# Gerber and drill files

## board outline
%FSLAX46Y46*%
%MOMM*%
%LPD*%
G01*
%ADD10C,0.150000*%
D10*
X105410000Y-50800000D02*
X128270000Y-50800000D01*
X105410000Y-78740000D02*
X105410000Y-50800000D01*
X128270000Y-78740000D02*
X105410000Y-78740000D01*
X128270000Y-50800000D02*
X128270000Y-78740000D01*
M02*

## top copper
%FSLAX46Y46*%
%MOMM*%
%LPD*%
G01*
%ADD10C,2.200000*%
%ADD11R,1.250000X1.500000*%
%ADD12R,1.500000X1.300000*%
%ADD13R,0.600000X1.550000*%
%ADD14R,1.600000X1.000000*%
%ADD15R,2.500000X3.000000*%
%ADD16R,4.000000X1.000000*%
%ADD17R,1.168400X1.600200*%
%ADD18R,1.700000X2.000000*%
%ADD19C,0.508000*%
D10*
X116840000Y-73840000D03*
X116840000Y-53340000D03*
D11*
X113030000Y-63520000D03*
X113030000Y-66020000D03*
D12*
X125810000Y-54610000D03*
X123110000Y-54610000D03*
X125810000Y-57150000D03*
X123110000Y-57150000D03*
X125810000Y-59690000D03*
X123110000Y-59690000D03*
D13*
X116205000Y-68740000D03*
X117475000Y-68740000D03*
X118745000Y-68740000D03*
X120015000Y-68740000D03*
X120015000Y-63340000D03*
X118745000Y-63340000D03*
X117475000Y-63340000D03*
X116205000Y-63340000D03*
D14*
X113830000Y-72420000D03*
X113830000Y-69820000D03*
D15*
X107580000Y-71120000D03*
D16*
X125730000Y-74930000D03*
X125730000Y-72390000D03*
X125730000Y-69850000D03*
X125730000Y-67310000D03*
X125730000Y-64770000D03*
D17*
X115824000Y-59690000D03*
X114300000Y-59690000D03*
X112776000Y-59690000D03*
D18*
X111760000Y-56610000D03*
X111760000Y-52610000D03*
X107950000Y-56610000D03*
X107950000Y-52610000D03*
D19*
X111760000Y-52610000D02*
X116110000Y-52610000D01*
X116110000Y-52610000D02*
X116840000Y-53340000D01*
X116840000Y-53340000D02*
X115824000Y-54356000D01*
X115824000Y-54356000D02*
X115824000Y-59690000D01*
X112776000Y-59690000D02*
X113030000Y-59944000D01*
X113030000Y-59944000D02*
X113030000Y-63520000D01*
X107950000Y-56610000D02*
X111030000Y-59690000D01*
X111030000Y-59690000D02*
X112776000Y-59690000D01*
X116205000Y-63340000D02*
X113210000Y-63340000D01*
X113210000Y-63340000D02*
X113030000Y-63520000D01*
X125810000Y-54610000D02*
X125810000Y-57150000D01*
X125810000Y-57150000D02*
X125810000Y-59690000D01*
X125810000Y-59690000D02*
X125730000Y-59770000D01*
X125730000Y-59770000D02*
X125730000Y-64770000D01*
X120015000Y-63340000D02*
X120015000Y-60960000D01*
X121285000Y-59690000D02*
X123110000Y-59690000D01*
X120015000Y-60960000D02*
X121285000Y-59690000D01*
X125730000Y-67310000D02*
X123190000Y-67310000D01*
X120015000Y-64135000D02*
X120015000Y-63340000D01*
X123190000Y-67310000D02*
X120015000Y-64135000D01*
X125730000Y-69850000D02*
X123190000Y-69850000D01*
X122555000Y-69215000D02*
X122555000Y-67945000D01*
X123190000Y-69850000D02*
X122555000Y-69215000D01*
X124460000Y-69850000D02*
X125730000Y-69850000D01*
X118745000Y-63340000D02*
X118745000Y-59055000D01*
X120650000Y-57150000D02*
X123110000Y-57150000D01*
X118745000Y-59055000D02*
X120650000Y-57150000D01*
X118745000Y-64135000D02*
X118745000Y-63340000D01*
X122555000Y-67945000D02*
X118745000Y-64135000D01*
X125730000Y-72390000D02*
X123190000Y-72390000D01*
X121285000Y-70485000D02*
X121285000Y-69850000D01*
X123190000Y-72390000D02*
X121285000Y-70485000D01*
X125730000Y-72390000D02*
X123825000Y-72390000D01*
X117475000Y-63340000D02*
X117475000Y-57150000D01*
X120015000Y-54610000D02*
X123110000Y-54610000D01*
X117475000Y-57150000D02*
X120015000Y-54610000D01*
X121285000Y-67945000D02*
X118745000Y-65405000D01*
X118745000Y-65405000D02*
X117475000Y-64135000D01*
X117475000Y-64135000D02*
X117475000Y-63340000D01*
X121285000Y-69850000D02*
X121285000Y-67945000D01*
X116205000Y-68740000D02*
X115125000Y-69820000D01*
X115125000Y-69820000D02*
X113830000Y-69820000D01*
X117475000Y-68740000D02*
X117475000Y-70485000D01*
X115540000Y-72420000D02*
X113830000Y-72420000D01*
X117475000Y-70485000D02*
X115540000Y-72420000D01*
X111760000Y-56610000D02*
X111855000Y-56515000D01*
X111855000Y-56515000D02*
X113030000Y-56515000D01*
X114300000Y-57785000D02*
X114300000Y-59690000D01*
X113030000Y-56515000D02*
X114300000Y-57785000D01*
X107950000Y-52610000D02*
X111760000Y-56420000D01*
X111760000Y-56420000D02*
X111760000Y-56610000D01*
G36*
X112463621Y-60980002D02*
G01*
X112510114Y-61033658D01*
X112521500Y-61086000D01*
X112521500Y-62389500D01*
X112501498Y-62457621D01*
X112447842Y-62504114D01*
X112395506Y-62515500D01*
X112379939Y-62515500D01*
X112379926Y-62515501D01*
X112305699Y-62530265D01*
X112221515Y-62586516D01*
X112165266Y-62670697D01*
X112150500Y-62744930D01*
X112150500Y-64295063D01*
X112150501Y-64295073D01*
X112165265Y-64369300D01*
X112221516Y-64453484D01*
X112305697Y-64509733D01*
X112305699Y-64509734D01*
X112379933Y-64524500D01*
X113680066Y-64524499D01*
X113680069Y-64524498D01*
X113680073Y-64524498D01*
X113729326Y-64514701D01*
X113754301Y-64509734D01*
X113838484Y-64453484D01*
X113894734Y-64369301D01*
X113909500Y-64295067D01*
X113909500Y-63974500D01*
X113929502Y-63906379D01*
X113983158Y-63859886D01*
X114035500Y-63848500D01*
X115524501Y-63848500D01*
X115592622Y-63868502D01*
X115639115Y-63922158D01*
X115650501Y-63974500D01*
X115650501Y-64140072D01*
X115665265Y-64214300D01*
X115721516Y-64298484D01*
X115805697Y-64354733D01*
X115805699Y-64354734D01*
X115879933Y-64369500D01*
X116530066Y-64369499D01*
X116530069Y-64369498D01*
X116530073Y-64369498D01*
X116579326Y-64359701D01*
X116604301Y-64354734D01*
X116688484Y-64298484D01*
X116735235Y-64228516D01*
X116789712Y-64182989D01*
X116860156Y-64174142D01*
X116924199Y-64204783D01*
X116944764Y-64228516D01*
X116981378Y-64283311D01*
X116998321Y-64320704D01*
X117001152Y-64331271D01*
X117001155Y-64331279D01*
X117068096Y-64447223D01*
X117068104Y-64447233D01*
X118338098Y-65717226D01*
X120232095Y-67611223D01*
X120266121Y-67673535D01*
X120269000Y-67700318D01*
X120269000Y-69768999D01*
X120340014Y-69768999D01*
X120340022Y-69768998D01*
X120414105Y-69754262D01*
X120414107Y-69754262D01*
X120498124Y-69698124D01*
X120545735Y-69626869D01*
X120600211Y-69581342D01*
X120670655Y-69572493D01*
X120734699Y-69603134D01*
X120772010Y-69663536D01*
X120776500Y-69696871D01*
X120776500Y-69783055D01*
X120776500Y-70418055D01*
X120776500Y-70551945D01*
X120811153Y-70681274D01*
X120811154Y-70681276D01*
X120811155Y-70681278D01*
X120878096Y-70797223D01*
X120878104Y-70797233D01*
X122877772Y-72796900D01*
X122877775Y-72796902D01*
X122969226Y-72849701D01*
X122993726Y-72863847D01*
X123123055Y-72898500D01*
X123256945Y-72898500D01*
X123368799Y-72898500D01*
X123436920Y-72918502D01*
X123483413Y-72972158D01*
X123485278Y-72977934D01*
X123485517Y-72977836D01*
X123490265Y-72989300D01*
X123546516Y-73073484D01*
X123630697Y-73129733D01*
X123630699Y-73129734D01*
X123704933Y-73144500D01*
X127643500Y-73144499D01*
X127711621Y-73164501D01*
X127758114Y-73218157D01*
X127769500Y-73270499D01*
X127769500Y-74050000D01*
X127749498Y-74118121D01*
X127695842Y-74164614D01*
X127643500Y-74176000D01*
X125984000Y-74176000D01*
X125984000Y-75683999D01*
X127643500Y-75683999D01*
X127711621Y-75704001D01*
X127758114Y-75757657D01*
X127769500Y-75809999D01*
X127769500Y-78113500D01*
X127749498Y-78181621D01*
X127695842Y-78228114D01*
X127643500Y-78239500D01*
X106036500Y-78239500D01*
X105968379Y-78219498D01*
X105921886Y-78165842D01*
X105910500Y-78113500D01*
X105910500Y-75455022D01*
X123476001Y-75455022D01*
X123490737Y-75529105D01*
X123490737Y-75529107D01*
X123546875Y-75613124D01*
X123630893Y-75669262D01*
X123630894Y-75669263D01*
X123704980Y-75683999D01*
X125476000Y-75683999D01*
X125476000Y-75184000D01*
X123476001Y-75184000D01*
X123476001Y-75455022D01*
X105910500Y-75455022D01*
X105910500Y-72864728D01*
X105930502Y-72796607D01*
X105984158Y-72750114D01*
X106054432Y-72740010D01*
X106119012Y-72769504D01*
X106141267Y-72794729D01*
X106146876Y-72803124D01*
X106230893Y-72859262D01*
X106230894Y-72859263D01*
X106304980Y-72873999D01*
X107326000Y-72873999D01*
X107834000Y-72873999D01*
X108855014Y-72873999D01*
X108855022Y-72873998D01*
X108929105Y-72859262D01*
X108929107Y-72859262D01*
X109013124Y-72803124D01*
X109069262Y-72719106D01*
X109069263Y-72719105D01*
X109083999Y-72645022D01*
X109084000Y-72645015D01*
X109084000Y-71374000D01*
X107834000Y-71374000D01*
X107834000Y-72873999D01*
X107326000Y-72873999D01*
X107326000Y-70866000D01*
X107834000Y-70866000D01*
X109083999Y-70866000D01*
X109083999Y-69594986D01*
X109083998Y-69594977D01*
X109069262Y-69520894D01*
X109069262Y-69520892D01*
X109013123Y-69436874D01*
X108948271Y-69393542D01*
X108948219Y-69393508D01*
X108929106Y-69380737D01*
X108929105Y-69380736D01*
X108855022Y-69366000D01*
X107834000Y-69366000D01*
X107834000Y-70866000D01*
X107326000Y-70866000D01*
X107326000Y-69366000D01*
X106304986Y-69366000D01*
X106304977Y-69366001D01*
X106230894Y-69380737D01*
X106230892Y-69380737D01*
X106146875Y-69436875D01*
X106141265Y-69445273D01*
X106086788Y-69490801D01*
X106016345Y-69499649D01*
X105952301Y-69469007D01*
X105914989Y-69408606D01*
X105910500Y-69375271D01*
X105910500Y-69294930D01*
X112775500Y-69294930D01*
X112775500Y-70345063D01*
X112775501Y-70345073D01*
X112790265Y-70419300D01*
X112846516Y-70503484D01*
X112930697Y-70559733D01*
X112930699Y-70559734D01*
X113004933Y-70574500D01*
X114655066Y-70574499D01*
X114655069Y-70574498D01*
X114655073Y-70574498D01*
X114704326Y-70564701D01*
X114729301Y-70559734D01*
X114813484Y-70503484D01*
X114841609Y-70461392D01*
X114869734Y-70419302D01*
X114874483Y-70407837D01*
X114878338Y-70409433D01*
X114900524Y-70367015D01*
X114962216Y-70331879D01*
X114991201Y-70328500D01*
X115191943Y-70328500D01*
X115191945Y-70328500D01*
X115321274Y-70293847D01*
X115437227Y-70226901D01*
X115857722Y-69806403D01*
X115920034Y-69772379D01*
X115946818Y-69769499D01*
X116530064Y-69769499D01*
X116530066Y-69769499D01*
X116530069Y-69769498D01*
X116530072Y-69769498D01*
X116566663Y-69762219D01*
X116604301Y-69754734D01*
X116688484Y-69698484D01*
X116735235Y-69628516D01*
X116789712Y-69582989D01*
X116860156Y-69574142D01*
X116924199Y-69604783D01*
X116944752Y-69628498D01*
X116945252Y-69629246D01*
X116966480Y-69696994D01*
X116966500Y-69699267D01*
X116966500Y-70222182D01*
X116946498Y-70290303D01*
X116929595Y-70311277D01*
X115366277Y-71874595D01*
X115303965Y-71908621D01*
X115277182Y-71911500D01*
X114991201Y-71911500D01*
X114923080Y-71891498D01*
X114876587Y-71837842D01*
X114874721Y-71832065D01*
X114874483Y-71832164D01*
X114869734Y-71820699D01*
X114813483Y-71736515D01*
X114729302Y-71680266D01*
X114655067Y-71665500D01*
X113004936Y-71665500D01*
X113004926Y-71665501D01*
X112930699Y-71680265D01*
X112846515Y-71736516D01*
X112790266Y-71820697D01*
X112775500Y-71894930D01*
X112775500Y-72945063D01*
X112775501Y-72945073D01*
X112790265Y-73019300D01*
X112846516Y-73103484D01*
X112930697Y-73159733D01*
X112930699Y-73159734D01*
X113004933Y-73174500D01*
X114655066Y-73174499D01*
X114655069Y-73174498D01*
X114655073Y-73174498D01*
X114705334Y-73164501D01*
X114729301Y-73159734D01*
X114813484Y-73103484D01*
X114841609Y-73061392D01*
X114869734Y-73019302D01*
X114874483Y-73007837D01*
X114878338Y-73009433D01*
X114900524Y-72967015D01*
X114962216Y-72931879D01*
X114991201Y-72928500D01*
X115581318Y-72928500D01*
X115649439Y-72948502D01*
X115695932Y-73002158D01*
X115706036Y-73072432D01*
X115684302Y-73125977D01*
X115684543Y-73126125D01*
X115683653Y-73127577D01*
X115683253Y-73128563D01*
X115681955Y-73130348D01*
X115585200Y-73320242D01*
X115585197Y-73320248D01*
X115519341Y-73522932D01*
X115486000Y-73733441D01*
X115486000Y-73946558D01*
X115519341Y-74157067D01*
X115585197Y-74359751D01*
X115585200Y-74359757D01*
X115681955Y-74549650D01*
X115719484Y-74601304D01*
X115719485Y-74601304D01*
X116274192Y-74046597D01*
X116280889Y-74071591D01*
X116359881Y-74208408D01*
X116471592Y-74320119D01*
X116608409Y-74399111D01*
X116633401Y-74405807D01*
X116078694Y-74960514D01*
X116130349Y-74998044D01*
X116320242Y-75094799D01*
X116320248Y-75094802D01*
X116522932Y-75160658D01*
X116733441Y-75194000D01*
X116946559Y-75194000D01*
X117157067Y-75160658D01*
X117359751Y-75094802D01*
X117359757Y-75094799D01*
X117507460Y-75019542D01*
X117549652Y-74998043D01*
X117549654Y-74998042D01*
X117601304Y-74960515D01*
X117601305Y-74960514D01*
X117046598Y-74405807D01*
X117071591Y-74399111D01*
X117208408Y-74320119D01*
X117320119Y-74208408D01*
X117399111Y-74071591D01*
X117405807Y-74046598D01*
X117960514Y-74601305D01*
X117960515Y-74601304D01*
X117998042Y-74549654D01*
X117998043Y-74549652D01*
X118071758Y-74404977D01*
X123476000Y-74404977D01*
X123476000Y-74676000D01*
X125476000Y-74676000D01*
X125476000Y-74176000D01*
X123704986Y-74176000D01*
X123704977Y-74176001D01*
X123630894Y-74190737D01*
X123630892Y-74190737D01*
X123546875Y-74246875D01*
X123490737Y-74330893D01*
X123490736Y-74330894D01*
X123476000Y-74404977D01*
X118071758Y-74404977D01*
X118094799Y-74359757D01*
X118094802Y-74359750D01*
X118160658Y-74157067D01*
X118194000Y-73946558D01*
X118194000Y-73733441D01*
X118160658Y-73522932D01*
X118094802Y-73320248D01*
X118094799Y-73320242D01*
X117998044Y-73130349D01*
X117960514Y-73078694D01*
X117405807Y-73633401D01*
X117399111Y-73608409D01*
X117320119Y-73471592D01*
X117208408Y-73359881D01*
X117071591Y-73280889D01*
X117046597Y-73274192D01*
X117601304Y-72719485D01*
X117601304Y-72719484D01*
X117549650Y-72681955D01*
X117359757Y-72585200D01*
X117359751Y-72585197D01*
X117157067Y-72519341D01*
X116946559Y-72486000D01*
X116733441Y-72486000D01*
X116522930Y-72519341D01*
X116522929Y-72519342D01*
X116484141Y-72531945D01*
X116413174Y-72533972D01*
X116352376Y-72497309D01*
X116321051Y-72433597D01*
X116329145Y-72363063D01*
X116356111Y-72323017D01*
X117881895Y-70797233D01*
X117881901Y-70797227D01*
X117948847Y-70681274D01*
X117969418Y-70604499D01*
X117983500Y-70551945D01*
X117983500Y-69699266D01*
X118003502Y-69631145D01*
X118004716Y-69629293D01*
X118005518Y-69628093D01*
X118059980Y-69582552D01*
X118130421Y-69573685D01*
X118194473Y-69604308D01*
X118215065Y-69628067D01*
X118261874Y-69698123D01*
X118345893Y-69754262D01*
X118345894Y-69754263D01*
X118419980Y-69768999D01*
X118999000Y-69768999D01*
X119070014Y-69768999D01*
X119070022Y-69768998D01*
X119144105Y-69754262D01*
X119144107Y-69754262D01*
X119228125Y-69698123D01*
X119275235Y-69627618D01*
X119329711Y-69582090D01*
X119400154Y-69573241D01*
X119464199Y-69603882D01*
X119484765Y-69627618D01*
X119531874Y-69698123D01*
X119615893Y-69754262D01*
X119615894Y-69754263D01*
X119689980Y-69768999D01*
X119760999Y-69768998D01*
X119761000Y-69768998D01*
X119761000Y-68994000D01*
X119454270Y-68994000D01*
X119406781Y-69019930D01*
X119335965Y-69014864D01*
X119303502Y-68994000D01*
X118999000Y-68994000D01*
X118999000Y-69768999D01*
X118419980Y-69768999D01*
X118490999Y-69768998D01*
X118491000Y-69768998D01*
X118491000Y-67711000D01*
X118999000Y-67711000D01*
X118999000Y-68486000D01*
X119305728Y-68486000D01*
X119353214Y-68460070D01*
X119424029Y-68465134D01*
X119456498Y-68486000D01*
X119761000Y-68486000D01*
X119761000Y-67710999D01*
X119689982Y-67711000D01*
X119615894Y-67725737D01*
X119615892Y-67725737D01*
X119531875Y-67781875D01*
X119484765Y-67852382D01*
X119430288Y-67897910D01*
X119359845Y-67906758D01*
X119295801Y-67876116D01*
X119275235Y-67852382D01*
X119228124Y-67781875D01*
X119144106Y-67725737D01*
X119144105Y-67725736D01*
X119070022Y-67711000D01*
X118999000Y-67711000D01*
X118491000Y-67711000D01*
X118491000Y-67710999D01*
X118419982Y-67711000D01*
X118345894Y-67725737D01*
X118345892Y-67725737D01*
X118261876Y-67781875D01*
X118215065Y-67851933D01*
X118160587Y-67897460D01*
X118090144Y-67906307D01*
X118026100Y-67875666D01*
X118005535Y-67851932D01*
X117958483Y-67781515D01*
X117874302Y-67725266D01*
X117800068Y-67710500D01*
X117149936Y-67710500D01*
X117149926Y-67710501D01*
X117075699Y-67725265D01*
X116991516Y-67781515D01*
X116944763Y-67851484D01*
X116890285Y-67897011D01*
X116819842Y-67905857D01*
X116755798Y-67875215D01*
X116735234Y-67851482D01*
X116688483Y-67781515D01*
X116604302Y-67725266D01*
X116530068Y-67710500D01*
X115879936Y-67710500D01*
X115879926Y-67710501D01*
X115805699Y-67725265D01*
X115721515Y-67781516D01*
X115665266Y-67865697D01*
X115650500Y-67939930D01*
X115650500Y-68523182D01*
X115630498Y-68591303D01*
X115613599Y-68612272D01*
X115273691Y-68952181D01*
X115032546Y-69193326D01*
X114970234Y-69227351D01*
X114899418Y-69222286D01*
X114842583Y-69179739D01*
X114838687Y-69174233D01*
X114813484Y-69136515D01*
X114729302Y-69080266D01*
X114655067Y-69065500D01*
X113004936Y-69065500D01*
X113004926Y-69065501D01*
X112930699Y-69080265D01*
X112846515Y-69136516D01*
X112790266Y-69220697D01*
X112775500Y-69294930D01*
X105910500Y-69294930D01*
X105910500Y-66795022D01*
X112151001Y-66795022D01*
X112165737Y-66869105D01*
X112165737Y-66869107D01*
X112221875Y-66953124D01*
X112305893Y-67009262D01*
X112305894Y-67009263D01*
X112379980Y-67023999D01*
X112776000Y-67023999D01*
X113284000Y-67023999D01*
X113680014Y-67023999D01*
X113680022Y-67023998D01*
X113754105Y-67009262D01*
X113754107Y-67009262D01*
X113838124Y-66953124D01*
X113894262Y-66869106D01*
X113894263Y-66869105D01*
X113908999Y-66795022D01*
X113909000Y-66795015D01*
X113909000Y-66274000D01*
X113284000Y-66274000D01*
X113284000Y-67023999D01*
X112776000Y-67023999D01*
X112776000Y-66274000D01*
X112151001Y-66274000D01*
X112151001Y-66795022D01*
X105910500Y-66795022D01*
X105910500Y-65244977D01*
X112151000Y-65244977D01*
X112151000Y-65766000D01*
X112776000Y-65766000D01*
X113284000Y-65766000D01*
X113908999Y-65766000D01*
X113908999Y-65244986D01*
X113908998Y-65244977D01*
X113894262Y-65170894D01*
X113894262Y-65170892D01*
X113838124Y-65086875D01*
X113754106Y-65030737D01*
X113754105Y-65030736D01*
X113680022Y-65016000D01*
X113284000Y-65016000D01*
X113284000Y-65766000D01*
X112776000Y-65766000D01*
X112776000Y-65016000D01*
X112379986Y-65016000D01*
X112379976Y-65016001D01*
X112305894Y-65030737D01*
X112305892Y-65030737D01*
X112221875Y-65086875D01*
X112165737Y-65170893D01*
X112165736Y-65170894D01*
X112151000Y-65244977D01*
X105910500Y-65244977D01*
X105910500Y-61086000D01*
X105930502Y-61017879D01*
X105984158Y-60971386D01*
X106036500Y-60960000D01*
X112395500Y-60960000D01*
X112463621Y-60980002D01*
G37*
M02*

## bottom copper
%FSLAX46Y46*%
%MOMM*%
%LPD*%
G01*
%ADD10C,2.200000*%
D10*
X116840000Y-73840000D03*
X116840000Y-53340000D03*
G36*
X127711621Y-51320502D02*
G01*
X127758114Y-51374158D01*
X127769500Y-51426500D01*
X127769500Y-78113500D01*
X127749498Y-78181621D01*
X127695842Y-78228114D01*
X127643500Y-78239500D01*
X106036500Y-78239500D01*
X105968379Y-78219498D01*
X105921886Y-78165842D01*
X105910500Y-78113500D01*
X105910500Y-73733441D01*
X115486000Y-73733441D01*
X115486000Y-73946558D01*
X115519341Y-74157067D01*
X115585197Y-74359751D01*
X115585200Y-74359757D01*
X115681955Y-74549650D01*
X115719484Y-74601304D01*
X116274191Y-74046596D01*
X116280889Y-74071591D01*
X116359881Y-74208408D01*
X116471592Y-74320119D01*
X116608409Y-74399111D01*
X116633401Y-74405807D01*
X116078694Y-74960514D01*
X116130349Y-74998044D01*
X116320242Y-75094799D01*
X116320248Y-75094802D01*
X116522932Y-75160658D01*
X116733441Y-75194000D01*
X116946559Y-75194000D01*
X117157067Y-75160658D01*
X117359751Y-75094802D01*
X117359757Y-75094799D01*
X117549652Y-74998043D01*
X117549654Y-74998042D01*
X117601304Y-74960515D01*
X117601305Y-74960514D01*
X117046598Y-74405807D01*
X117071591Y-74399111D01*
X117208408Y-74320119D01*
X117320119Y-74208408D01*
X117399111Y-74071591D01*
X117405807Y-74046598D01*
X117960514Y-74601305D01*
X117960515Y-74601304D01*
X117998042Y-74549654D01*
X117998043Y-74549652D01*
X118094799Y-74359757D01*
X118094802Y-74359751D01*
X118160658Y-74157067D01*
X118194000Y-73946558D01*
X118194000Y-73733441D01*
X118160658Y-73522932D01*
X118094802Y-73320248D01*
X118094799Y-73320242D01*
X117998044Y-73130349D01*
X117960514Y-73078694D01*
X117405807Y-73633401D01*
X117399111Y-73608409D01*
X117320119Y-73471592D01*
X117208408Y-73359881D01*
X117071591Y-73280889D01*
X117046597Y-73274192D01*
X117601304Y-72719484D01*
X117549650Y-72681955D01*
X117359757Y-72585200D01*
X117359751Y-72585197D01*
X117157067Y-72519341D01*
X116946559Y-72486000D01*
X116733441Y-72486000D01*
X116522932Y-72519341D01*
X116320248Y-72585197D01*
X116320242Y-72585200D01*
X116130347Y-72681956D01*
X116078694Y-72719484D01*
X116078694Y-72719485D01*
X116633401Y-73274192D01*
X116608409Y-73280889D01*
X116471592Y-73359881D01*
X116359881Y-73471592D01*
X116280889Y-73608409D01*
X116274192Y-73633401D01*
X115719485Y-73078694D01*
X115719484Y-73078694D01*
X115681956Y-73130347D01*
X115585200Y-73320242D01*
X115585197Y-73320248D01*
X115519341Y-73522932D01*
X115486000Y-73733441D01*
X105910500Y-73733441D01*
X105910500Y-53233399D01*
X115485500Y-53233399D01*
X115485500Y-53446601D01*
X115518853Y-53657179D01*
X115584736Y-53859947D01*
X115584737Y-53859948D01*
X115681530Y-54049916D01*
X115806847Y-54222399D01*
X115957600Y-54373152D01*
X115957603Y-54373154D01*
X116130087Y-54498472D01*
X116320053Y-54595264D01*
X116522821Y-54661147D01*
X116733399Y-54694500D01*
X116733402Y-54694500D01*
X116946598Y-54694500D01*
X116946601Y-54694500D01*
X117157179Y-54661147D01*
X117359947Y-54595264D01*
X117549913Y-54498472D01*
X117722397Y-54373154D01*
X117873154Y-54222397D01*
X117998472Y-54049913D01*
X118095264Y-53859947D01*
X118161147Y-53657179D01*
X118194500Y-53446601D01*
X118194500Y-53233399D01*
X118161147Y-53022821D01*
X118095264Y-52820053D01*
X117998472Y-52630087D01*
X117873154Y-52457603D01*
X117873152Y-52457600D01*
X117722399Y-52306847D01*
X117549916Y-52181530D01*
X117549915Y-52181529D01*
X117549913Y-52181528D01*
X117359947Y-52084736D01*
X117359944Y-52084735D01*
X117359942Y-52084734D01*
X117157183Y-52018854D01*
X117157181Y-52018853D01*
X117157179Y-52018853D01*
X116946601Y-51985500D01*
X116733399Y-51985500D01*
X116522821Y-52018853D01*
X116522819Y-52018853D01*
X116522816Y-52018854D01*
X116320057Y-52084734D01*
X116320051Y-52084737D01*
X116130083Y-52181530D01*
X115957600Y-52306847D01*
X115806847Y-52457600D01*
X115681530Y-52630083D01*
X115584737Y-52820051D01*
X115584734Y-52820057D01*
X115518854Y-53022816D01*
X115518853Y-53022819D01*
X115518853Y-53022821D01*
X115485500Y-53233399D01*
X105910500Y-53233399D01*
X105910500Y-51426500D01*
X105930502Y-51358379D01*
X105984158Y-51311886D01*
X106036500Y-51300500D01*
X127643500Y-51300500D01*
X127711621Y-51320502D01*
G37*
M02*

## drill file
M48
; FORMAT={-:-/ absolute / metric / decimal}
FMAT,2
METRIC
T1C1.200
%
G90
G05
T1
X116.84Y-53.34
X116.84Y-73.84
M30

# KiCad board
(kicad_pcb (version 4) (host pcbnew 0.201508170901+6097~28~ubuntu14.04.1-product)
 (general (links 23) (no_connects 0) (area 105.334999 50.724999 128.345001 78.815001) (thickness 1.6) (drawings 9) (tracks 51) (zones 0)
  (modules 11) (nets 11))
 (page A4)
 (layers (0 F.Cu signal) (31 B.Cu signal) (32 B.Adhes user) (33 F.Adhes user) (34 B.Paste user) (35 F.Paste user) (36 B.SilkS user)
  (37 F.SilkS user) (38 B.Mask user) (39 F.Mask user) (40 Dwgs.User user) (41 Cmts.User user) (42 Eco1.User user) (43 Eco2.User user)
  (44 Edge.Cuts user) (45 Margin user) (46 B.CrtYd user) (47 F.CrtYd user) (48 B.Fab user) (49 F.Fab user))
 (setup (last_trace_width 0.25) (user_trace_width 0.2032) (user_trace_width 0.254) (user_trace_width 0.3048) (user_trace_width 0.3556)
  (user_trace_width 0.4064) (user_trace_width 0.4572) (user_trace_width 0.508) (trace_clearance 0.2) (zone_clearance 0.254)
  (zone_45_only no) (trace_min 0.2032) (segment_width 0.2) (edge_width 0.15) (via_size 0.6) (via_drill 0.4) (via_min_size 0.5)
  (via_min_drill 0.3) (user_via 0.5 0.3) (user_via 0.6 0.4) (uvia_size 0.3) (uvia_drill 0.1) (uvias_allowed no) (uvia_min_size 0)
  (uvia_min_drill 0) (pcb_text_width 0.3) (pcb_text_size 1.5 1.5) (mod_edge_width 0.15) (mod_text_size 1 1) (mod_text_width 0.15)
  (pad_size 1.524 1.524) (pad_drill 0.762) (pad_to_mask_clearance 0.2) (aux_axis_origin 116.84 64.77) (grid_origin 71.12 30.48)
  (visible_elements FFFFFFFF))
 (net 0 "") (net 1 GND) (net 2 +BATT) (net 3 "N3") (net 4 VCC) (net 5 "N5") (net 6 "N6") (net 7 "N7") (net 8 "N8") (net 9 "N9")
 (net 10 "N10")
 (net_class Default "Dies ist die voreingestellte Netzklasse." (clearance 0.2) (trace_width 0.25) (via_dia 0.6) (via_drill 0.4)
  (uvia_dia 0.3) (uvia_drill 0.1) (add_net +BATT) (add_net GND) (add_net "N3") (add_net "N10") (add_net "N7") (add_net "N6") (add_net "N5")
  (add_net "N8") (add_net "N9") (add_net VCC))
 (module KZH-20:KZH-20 (layer B.Cu) (at 116.84 53.34 90)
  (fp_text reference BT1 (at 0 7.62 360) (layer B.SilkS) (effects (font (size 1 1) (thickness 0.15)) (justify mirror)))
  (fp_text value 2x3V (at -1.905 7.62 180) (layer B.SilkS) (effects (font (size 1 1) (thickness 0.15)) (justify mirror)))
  (pad 2 thru_hole circle (at -20.5 0 90) (size 2.2 2.2) (drill 1.2) (layers *.Cu *.Mask B.SilkS) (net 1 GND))
  (pad 1 thru_hole circle (at 0 0 90) (size 2.2 2.2) (drill 1.2) (layers *.Cu *.Mask B.SilkS) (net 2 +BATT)))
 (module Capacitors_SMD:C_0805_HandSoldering (layer F.Cu) (at 113.03 64.77 270)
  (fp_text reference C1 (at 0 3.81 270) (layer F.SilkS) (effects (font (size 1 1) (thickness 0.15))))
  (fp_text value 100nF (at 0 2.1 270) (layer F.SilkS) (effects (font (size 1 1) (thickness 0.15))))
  (pad 1 smd rect (at -1.25 0 270) (size 1.5 1.25) (layers F.Cu F.Paste F.Mask) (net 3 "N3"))
  (pad 2 smd rect (at 1.25 0 270) (size 1.5 1.25) (layers F.Cu F.Paste F.Mask) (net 1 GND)))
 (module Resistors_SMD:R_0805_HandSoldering (layer F.Cu) (at 124.46 54.61 180)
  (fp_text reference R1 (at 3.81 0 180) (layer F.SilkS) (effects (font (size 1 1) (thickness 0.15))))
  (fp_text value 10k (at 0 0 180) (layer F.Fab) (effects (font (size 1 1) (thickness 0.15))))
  (pad 1 smd rect (at -1.35 0 180) (size 1.5 1.3) (layers F.Cu F.Paste F.Mask) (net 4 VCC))
  (pad 2 smd rect (at 1.35 0 180) (size 1.5 1.3) (layers F.Cu F.Paste F.Mask) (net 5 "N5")))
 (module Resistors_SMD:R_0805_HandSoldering (layer F.Cu) (at 124.46 57.15 180)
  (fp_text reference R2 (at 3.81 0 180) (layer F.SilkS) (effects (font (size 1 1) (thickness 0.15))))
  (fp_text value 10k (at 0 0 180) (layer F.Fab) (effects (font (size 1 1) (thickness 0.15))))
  (pad 1 smd rect (at -1.35 0 180) (size 1.5 1.3) (layers F.Cu F.Paste F.Mask) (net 4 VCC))
  (pad 2 smd rect (at 1.35 0 180) (size 1.5 1.3) (layers F.Cu F.Paste F.Mask) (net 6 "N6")))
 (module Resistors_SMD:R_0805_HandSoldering (layer F.Cu) (at 124.46 59.69 180)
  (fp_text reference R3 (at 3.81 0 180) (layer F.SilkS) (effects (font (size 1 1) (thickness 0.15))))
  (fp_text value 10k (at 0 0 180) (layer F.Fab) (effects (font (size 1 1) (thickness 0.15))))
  (pad 1 smd rect (at -1.35 0 180) (size 1.5 1.3) (layers F.Cu F.Paste F.Mask) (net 4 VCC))
  (pad 2 smd rect (at 1.35 0 180) (size 1.5 1.3) (layers F.Cu F.Paste F.Mask) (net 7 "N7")))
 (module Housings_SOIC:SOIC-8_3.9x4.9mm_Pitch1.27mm (layer F.Cu) (at 118.11 66.04 90)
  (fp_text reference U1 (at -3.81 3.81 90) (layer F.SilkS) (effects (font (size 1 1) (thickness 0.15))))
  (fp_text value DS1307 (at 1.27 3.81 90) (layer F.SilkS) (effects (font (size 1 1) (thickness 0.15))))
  (pad 1 smd rect (at -2.7 -1.905 90) (size 1.55 0.6) (layers F.Cu F.Paste F.Mask) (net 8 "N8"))
  (pad 2 smd rect (at -2.7 -0.635 90) (size 1.55 0.6) (layers F.Cu F.Paste F.Mask) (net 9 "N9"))
  (pad 3 smd rect (at -2.7 0.635 90) (size 1.55 0.6) (layers F.Cu F.Paste F.Mask) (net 1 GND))
  (pad 4 smd rect (at -2.7 1.905 90) (size 1.55 0.6) (layers F.Cu F.Paste F.Mask) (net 1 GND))
  (pad 5 smd rect (at 2.7 1.905 90) (size 1.55 0.6) (layers F.Cu F.Paste F.Mask) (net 7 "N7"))
  (pad 6 smd rect (at 2.7 0.635 90) (size 1.55 0.6) (layers F.Cu F.Paste F.Mask) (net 6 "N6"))
  (pad 7 smd rect (at 2.7 -0.635 90) (size 1.55 0.6) (layers F.Cu F.Paste F.Mask) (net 5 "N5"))
  (pad 8 smd rect (at 2.7 -1.905 90) (size 1.55 0.6) (layers F.Cu F.Paste F.Mask) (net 3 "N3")))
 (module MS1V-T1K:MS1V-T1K (layer F.Cu) (at 113.03 71.12)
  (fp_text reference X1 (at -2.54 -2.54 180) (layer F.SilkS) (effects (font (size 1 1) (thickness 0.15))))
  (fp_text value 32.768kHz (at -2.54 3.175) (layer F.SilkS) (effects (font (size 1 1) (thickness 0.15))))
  (pad 1 smd rect (at 0.8 1.3) (size 1.6 1) (layers F.Cu F.Paste F.Mask) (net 9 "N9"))
  (pad 2 smd rect (at 0.8 -1.3) (size 1.6 1) (layers F.Cu F.Paste F.Mask) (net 8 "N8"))
  (pad 3 smd rect (at -5.45 0) (size 2.5 3) (layers F.Cu F.Paste F.Mask) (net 1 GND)))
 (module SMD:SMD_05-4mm (layer F.Cu) (at 125.73 64.77)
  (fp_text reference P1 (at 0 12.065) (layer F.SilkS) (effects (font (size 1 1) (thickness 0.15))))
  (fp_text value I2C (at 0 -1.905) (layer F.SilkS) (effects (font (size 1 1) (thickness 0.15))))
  (pad 5 connect rect (at 0 10.16) (size 4 1) (layers F.Cu F.Mask) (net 1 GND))
  (pad 4 connect rect (at 0 7.62) (size 4 1) (layers F.Cu F.Mask) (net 5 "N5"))
  (pad 3 connect rect (at 0 5.08) (size 4 1) (layers F.Cu F.Mask) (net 6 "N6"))
  (pad 2 connect rect (at 0 2.54) (size 4 1) (layers F.Cu F.Mask) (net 7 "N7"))
  (pad 1 connect rect (at 0 0) (size 4 1) (layers F.Cu F.Mask) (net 4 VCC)))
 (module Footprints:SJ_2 (layer F.Cu) (at 114.3 59.69 180)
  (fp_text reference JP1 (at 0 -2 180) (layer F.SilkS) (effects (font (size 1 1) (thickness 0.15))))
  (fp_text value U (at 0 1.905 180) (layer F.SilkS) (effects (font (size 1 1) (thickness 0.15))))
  (pad 1 smd rect (at -1.524 0 180) (size 1.1684 1.6002) (layers F.Cu F.Paste F.Mask) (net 2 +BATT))
  (pad 2 smd rect (at 0 0 180) (size 1.1684 1.6002) (layers F.Cu F.Paste F.Mask) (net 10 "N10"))
  (pad 3 smd rect (at 1.524 0 180) (size 1.1684 1.6002) (layers F.Cu F.Paste F.Mask) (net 3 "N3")))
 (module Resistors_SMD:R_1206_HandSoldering (layer F.Cu) (at 111.76 54.61 90)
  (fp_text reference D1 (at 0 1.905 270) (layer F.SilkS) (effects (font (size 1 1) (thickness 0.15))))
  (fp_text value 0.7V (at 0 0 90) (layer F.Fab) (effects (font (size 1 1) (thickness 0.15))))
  (pad 1 smd rect (at -2 0 90) (size 2 1.7) (layers F.Cu F.Paste F.Mask) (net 10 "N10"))
  (pad 2 smd rect (at 2 0 90) (size 2 1.7) (layers F.Cu F.Paste F.Mask) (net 2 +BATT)))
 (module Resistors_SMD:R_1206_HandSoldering (layer F.Cu) (at 107.95 54.61 90)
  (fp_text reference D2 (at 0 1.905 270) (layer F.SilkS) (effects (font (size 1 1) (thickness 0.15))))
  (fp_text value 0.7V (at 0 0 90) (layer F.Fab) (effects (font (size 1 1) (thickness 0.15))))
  (pad 1 smd rect (at -2 0 90) (size 2 1.7) (layers F.Cu F.Paste F.Mask) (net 3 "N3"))
  (pad 2 smd rect (at 2 0 90) (size 2 1.7) (layers F.Cu F.Paste F.Mask) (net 10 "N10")))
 (gr_line (start 105.41 50.8) (end 128.27 50.8) (angle 90) (layer Edge.Cuts) (width 0.15))
 (gr_line (start 105.41 78.74) (end 105.41 50.8) (angle 90) (layer Edge.Cuts) (width 0.15))
 (gr_line (start 128.27 78.74) (end 105.41 78.74) (angle 90) (layer Edge.Cuts) (width 0.15))
 (gr_line (start 128.27 50.8) (end 128.27 78.74) (angle 90) (layer Edge.Cuts) (width 0.15))
 (segment (start 111.76 52.61) (end 116.11 52.61) (width 0.508) (layer F.Cu) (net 2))
 (segment (start 116.11 52.61) (end 116.84 53.34) (width 0.508) (layer F.Cu) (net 2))
 (segment (start 116.84 53.34) (end 115.824 54.356) (width 0.508) (layer F.Cu) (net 2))
 (segment (start 115.824 54.356) (end 115.824 59.69) (width 0.508) (layer F.Cu) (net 2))
 (segment (start 112.776 59.69) (end 113.03 59.944) (width 0.508) (layer F.Cu) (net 3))
 (segment (start 113.03 59.944) (end 113.03 63.52) (width 0.508) (layer F.Cu) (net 3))
 (segment (start 107.95 56.61) (end 111.03 59.69) (width 0.508) (layer F.Cu) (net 3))
 (segment (start 111.03 59.69) (end 112.776 59.69) (width 0.508) (layer F.Cu) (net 3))
 (segment (start 116.205 63.34) (end 113.21 63.34) (width 0.508) (layer F.Cu) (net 3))
 (segment (start 113.21 63.34) (end 113.03 63.52) (width 0.508) (layer F.Cu) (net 3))
 (segment (start 125.81 54.61) (end 125.81 57.15) (width 0.508) (layer F.Cu) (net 4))
 (segment (start 125.81 57.15) (end 125.81 59.69) (width 0.508) (layer F.Cu) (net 4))
 (segment (start 125.81 59.69) (end 125.73 59.77) (width 0.508) (layer F.Cu) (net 4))
 (segment (start 125.73 59.77) (end 125.73 64.77) (width 0.508) (layer F.Cu) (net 4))
 (segment (start 120.015 63.34) (end 120.015 60.96) (width 0.508) (layer F.Cu) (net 7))
 (segment (start 121.285 59.69) (end 123.11 59.69) (width 0.508) (layer F.Cu) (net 7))
 (segment (start 120.015 60.96) (end 121.285 59.69) (width 0.508) (layer F.Cu) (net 7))
 (segment (start 125.73 67.31) (end 123.19 67.31) (width 0.508) (layer F.Cu) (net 7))
 (segment (start 120.015 64.135) (end 120.015 63.34) (width 0.508) (layer F.Cu) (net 7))
 (segment (start 123.19 67.31) (end 120.015 64.135) (width 0.508) (layer F.Cu) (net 7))
 (segment (start 125.73 69.85) (end 123.19 69.85) (width 0.508) (layer F.Cu) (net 6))
 (segment (start 122.555 69.215) (end 122.555 67.945) (width 0.508) (layer F.Cu) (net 6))
 (segment (start 123.19 69.85) (end 122.555 69.215) (width 0.508) (layer F.Cu) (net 6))
 (segment (start 124.46 69.85) (end 125.73 69.85) (width 0.508) (layer F.Cu) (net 6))
 (segment (start 118.745 63.34) (end 118.745 59.055) (width 0.508) (layer F.Cu) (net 6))
 (segment (start 120.65 57.15) (end 123.11 57.15) (width 0.508) (layer F.Cu) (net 6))
 (segment (start 118.745 59.055) (end 120.65 57.15) (width 0.508) (layer F.Cu) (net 6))
 (segment (start 118.745 64.135) (end 118.745 63.34) (width 0.508) (layer F.Cu) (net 6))
 (segment (start 122.555 67.945) (end 118.745 64.135) (width 0.508) (layer F.Cu) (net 6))
 (segment (start 125.73 72.39) (end 123.19 72.39) (width 0.508) (layer F.Cu) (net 5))
 (segment (start 121.285 70.485) (end 121.285 69.85) (width 0.508) (layer F.Cu) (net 5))
 (segment (start 123.19 72.39) (end 121.285 70.485) (width 0.508) (layer F.Cu) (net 5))
 (segment (start 125.73 72.39) (end 123.825 72.39) (width 0.508) (layer F.Cu) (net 5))
 (segment (start 117.475 63.34) (end 117.475 57.15) (width 0.508) (layer F.Cu) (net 5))
 (segment (start 120.015 54.61) (end 123.11 54.61) (width 0.508) (layer F.Cu) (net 5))
 (segment (start 117.475 57.15) (end 120.015 54.61) (width 0.508) (layer F.Cu) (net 5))
 (segment (start 121.285 67.945) (end 118.745 65.405) (width 0.508) (layer F.Cu) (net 5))
 (segment (start 118.745 65.405) (end 117.475 64.135) (width 0.508) (layer F.Cu) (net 5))
 (segment (start 117.475 64.135) (end 117.475 63.34) (width 0.508) (layer F.Cu) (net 5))
 (segment (start 121.285 69.85) (end 121.285 67.945) (width 0.508) (layer F.Cu) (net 5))
 (segment (start 116.205 68.74) (end 115.125 69.82) (width 0.508) (layer F.Cu) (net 8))
 (segment (start 115.125 69.82) (end 113.83 69.82) (width 0.508) (layer F.Cu) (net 8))
 (segment (start 117.475 68.74) (end 117.475 70.485) (width 0.508) (layer F.Cu) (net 9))
 (segment (start 115.54 72.42) (end 113.83 72.42) (width 0.508) (layer F.Cu) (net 9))
 (segment (start 117.475 70.485) (end 115.54 72.42) (width 0.508) (layer F.Cu) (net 9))
 (segment (start 111.76 56.61) (end 111.855 56.515) (width 0.508) (layer F.Cu) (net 10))
 (segment (start 111.855 56.515) (end 113.03 56.515) (width 0.508) (layer F.Cu) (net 10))
 (segment (start 114.3 57.785) (end 114.3 59.69) (width 0.508) (layer F.Cu) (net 10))
 (segment (start 113.03 56.515) (end 114.3 57.785) (width 0.508) (layer F.Cu) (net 10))
 (segment (start 107.95 52.61) (end 111.76 56.42) (width 0.508) (layer F.Cu) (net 10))
 (segment (start 111.76 56.42) (end 111.76 56.61) (width 0.508) (layer F.Cu) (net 10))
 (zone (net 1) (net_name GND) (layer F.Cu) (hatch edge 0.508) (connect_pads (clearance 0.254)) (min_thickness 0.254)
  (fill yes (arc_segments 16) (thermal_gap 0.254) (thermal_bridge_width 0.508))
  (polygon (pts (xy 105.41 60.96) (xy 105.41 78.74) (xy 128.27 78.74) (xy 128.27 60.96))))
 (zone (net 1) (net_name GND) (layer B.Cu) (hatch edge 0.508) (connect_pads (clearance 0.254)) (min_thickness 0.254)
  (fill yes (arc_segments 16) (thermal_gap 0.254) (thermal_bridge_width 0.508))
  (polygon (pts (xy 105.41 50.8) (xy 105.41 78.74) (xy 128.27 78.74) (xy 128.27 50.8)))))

